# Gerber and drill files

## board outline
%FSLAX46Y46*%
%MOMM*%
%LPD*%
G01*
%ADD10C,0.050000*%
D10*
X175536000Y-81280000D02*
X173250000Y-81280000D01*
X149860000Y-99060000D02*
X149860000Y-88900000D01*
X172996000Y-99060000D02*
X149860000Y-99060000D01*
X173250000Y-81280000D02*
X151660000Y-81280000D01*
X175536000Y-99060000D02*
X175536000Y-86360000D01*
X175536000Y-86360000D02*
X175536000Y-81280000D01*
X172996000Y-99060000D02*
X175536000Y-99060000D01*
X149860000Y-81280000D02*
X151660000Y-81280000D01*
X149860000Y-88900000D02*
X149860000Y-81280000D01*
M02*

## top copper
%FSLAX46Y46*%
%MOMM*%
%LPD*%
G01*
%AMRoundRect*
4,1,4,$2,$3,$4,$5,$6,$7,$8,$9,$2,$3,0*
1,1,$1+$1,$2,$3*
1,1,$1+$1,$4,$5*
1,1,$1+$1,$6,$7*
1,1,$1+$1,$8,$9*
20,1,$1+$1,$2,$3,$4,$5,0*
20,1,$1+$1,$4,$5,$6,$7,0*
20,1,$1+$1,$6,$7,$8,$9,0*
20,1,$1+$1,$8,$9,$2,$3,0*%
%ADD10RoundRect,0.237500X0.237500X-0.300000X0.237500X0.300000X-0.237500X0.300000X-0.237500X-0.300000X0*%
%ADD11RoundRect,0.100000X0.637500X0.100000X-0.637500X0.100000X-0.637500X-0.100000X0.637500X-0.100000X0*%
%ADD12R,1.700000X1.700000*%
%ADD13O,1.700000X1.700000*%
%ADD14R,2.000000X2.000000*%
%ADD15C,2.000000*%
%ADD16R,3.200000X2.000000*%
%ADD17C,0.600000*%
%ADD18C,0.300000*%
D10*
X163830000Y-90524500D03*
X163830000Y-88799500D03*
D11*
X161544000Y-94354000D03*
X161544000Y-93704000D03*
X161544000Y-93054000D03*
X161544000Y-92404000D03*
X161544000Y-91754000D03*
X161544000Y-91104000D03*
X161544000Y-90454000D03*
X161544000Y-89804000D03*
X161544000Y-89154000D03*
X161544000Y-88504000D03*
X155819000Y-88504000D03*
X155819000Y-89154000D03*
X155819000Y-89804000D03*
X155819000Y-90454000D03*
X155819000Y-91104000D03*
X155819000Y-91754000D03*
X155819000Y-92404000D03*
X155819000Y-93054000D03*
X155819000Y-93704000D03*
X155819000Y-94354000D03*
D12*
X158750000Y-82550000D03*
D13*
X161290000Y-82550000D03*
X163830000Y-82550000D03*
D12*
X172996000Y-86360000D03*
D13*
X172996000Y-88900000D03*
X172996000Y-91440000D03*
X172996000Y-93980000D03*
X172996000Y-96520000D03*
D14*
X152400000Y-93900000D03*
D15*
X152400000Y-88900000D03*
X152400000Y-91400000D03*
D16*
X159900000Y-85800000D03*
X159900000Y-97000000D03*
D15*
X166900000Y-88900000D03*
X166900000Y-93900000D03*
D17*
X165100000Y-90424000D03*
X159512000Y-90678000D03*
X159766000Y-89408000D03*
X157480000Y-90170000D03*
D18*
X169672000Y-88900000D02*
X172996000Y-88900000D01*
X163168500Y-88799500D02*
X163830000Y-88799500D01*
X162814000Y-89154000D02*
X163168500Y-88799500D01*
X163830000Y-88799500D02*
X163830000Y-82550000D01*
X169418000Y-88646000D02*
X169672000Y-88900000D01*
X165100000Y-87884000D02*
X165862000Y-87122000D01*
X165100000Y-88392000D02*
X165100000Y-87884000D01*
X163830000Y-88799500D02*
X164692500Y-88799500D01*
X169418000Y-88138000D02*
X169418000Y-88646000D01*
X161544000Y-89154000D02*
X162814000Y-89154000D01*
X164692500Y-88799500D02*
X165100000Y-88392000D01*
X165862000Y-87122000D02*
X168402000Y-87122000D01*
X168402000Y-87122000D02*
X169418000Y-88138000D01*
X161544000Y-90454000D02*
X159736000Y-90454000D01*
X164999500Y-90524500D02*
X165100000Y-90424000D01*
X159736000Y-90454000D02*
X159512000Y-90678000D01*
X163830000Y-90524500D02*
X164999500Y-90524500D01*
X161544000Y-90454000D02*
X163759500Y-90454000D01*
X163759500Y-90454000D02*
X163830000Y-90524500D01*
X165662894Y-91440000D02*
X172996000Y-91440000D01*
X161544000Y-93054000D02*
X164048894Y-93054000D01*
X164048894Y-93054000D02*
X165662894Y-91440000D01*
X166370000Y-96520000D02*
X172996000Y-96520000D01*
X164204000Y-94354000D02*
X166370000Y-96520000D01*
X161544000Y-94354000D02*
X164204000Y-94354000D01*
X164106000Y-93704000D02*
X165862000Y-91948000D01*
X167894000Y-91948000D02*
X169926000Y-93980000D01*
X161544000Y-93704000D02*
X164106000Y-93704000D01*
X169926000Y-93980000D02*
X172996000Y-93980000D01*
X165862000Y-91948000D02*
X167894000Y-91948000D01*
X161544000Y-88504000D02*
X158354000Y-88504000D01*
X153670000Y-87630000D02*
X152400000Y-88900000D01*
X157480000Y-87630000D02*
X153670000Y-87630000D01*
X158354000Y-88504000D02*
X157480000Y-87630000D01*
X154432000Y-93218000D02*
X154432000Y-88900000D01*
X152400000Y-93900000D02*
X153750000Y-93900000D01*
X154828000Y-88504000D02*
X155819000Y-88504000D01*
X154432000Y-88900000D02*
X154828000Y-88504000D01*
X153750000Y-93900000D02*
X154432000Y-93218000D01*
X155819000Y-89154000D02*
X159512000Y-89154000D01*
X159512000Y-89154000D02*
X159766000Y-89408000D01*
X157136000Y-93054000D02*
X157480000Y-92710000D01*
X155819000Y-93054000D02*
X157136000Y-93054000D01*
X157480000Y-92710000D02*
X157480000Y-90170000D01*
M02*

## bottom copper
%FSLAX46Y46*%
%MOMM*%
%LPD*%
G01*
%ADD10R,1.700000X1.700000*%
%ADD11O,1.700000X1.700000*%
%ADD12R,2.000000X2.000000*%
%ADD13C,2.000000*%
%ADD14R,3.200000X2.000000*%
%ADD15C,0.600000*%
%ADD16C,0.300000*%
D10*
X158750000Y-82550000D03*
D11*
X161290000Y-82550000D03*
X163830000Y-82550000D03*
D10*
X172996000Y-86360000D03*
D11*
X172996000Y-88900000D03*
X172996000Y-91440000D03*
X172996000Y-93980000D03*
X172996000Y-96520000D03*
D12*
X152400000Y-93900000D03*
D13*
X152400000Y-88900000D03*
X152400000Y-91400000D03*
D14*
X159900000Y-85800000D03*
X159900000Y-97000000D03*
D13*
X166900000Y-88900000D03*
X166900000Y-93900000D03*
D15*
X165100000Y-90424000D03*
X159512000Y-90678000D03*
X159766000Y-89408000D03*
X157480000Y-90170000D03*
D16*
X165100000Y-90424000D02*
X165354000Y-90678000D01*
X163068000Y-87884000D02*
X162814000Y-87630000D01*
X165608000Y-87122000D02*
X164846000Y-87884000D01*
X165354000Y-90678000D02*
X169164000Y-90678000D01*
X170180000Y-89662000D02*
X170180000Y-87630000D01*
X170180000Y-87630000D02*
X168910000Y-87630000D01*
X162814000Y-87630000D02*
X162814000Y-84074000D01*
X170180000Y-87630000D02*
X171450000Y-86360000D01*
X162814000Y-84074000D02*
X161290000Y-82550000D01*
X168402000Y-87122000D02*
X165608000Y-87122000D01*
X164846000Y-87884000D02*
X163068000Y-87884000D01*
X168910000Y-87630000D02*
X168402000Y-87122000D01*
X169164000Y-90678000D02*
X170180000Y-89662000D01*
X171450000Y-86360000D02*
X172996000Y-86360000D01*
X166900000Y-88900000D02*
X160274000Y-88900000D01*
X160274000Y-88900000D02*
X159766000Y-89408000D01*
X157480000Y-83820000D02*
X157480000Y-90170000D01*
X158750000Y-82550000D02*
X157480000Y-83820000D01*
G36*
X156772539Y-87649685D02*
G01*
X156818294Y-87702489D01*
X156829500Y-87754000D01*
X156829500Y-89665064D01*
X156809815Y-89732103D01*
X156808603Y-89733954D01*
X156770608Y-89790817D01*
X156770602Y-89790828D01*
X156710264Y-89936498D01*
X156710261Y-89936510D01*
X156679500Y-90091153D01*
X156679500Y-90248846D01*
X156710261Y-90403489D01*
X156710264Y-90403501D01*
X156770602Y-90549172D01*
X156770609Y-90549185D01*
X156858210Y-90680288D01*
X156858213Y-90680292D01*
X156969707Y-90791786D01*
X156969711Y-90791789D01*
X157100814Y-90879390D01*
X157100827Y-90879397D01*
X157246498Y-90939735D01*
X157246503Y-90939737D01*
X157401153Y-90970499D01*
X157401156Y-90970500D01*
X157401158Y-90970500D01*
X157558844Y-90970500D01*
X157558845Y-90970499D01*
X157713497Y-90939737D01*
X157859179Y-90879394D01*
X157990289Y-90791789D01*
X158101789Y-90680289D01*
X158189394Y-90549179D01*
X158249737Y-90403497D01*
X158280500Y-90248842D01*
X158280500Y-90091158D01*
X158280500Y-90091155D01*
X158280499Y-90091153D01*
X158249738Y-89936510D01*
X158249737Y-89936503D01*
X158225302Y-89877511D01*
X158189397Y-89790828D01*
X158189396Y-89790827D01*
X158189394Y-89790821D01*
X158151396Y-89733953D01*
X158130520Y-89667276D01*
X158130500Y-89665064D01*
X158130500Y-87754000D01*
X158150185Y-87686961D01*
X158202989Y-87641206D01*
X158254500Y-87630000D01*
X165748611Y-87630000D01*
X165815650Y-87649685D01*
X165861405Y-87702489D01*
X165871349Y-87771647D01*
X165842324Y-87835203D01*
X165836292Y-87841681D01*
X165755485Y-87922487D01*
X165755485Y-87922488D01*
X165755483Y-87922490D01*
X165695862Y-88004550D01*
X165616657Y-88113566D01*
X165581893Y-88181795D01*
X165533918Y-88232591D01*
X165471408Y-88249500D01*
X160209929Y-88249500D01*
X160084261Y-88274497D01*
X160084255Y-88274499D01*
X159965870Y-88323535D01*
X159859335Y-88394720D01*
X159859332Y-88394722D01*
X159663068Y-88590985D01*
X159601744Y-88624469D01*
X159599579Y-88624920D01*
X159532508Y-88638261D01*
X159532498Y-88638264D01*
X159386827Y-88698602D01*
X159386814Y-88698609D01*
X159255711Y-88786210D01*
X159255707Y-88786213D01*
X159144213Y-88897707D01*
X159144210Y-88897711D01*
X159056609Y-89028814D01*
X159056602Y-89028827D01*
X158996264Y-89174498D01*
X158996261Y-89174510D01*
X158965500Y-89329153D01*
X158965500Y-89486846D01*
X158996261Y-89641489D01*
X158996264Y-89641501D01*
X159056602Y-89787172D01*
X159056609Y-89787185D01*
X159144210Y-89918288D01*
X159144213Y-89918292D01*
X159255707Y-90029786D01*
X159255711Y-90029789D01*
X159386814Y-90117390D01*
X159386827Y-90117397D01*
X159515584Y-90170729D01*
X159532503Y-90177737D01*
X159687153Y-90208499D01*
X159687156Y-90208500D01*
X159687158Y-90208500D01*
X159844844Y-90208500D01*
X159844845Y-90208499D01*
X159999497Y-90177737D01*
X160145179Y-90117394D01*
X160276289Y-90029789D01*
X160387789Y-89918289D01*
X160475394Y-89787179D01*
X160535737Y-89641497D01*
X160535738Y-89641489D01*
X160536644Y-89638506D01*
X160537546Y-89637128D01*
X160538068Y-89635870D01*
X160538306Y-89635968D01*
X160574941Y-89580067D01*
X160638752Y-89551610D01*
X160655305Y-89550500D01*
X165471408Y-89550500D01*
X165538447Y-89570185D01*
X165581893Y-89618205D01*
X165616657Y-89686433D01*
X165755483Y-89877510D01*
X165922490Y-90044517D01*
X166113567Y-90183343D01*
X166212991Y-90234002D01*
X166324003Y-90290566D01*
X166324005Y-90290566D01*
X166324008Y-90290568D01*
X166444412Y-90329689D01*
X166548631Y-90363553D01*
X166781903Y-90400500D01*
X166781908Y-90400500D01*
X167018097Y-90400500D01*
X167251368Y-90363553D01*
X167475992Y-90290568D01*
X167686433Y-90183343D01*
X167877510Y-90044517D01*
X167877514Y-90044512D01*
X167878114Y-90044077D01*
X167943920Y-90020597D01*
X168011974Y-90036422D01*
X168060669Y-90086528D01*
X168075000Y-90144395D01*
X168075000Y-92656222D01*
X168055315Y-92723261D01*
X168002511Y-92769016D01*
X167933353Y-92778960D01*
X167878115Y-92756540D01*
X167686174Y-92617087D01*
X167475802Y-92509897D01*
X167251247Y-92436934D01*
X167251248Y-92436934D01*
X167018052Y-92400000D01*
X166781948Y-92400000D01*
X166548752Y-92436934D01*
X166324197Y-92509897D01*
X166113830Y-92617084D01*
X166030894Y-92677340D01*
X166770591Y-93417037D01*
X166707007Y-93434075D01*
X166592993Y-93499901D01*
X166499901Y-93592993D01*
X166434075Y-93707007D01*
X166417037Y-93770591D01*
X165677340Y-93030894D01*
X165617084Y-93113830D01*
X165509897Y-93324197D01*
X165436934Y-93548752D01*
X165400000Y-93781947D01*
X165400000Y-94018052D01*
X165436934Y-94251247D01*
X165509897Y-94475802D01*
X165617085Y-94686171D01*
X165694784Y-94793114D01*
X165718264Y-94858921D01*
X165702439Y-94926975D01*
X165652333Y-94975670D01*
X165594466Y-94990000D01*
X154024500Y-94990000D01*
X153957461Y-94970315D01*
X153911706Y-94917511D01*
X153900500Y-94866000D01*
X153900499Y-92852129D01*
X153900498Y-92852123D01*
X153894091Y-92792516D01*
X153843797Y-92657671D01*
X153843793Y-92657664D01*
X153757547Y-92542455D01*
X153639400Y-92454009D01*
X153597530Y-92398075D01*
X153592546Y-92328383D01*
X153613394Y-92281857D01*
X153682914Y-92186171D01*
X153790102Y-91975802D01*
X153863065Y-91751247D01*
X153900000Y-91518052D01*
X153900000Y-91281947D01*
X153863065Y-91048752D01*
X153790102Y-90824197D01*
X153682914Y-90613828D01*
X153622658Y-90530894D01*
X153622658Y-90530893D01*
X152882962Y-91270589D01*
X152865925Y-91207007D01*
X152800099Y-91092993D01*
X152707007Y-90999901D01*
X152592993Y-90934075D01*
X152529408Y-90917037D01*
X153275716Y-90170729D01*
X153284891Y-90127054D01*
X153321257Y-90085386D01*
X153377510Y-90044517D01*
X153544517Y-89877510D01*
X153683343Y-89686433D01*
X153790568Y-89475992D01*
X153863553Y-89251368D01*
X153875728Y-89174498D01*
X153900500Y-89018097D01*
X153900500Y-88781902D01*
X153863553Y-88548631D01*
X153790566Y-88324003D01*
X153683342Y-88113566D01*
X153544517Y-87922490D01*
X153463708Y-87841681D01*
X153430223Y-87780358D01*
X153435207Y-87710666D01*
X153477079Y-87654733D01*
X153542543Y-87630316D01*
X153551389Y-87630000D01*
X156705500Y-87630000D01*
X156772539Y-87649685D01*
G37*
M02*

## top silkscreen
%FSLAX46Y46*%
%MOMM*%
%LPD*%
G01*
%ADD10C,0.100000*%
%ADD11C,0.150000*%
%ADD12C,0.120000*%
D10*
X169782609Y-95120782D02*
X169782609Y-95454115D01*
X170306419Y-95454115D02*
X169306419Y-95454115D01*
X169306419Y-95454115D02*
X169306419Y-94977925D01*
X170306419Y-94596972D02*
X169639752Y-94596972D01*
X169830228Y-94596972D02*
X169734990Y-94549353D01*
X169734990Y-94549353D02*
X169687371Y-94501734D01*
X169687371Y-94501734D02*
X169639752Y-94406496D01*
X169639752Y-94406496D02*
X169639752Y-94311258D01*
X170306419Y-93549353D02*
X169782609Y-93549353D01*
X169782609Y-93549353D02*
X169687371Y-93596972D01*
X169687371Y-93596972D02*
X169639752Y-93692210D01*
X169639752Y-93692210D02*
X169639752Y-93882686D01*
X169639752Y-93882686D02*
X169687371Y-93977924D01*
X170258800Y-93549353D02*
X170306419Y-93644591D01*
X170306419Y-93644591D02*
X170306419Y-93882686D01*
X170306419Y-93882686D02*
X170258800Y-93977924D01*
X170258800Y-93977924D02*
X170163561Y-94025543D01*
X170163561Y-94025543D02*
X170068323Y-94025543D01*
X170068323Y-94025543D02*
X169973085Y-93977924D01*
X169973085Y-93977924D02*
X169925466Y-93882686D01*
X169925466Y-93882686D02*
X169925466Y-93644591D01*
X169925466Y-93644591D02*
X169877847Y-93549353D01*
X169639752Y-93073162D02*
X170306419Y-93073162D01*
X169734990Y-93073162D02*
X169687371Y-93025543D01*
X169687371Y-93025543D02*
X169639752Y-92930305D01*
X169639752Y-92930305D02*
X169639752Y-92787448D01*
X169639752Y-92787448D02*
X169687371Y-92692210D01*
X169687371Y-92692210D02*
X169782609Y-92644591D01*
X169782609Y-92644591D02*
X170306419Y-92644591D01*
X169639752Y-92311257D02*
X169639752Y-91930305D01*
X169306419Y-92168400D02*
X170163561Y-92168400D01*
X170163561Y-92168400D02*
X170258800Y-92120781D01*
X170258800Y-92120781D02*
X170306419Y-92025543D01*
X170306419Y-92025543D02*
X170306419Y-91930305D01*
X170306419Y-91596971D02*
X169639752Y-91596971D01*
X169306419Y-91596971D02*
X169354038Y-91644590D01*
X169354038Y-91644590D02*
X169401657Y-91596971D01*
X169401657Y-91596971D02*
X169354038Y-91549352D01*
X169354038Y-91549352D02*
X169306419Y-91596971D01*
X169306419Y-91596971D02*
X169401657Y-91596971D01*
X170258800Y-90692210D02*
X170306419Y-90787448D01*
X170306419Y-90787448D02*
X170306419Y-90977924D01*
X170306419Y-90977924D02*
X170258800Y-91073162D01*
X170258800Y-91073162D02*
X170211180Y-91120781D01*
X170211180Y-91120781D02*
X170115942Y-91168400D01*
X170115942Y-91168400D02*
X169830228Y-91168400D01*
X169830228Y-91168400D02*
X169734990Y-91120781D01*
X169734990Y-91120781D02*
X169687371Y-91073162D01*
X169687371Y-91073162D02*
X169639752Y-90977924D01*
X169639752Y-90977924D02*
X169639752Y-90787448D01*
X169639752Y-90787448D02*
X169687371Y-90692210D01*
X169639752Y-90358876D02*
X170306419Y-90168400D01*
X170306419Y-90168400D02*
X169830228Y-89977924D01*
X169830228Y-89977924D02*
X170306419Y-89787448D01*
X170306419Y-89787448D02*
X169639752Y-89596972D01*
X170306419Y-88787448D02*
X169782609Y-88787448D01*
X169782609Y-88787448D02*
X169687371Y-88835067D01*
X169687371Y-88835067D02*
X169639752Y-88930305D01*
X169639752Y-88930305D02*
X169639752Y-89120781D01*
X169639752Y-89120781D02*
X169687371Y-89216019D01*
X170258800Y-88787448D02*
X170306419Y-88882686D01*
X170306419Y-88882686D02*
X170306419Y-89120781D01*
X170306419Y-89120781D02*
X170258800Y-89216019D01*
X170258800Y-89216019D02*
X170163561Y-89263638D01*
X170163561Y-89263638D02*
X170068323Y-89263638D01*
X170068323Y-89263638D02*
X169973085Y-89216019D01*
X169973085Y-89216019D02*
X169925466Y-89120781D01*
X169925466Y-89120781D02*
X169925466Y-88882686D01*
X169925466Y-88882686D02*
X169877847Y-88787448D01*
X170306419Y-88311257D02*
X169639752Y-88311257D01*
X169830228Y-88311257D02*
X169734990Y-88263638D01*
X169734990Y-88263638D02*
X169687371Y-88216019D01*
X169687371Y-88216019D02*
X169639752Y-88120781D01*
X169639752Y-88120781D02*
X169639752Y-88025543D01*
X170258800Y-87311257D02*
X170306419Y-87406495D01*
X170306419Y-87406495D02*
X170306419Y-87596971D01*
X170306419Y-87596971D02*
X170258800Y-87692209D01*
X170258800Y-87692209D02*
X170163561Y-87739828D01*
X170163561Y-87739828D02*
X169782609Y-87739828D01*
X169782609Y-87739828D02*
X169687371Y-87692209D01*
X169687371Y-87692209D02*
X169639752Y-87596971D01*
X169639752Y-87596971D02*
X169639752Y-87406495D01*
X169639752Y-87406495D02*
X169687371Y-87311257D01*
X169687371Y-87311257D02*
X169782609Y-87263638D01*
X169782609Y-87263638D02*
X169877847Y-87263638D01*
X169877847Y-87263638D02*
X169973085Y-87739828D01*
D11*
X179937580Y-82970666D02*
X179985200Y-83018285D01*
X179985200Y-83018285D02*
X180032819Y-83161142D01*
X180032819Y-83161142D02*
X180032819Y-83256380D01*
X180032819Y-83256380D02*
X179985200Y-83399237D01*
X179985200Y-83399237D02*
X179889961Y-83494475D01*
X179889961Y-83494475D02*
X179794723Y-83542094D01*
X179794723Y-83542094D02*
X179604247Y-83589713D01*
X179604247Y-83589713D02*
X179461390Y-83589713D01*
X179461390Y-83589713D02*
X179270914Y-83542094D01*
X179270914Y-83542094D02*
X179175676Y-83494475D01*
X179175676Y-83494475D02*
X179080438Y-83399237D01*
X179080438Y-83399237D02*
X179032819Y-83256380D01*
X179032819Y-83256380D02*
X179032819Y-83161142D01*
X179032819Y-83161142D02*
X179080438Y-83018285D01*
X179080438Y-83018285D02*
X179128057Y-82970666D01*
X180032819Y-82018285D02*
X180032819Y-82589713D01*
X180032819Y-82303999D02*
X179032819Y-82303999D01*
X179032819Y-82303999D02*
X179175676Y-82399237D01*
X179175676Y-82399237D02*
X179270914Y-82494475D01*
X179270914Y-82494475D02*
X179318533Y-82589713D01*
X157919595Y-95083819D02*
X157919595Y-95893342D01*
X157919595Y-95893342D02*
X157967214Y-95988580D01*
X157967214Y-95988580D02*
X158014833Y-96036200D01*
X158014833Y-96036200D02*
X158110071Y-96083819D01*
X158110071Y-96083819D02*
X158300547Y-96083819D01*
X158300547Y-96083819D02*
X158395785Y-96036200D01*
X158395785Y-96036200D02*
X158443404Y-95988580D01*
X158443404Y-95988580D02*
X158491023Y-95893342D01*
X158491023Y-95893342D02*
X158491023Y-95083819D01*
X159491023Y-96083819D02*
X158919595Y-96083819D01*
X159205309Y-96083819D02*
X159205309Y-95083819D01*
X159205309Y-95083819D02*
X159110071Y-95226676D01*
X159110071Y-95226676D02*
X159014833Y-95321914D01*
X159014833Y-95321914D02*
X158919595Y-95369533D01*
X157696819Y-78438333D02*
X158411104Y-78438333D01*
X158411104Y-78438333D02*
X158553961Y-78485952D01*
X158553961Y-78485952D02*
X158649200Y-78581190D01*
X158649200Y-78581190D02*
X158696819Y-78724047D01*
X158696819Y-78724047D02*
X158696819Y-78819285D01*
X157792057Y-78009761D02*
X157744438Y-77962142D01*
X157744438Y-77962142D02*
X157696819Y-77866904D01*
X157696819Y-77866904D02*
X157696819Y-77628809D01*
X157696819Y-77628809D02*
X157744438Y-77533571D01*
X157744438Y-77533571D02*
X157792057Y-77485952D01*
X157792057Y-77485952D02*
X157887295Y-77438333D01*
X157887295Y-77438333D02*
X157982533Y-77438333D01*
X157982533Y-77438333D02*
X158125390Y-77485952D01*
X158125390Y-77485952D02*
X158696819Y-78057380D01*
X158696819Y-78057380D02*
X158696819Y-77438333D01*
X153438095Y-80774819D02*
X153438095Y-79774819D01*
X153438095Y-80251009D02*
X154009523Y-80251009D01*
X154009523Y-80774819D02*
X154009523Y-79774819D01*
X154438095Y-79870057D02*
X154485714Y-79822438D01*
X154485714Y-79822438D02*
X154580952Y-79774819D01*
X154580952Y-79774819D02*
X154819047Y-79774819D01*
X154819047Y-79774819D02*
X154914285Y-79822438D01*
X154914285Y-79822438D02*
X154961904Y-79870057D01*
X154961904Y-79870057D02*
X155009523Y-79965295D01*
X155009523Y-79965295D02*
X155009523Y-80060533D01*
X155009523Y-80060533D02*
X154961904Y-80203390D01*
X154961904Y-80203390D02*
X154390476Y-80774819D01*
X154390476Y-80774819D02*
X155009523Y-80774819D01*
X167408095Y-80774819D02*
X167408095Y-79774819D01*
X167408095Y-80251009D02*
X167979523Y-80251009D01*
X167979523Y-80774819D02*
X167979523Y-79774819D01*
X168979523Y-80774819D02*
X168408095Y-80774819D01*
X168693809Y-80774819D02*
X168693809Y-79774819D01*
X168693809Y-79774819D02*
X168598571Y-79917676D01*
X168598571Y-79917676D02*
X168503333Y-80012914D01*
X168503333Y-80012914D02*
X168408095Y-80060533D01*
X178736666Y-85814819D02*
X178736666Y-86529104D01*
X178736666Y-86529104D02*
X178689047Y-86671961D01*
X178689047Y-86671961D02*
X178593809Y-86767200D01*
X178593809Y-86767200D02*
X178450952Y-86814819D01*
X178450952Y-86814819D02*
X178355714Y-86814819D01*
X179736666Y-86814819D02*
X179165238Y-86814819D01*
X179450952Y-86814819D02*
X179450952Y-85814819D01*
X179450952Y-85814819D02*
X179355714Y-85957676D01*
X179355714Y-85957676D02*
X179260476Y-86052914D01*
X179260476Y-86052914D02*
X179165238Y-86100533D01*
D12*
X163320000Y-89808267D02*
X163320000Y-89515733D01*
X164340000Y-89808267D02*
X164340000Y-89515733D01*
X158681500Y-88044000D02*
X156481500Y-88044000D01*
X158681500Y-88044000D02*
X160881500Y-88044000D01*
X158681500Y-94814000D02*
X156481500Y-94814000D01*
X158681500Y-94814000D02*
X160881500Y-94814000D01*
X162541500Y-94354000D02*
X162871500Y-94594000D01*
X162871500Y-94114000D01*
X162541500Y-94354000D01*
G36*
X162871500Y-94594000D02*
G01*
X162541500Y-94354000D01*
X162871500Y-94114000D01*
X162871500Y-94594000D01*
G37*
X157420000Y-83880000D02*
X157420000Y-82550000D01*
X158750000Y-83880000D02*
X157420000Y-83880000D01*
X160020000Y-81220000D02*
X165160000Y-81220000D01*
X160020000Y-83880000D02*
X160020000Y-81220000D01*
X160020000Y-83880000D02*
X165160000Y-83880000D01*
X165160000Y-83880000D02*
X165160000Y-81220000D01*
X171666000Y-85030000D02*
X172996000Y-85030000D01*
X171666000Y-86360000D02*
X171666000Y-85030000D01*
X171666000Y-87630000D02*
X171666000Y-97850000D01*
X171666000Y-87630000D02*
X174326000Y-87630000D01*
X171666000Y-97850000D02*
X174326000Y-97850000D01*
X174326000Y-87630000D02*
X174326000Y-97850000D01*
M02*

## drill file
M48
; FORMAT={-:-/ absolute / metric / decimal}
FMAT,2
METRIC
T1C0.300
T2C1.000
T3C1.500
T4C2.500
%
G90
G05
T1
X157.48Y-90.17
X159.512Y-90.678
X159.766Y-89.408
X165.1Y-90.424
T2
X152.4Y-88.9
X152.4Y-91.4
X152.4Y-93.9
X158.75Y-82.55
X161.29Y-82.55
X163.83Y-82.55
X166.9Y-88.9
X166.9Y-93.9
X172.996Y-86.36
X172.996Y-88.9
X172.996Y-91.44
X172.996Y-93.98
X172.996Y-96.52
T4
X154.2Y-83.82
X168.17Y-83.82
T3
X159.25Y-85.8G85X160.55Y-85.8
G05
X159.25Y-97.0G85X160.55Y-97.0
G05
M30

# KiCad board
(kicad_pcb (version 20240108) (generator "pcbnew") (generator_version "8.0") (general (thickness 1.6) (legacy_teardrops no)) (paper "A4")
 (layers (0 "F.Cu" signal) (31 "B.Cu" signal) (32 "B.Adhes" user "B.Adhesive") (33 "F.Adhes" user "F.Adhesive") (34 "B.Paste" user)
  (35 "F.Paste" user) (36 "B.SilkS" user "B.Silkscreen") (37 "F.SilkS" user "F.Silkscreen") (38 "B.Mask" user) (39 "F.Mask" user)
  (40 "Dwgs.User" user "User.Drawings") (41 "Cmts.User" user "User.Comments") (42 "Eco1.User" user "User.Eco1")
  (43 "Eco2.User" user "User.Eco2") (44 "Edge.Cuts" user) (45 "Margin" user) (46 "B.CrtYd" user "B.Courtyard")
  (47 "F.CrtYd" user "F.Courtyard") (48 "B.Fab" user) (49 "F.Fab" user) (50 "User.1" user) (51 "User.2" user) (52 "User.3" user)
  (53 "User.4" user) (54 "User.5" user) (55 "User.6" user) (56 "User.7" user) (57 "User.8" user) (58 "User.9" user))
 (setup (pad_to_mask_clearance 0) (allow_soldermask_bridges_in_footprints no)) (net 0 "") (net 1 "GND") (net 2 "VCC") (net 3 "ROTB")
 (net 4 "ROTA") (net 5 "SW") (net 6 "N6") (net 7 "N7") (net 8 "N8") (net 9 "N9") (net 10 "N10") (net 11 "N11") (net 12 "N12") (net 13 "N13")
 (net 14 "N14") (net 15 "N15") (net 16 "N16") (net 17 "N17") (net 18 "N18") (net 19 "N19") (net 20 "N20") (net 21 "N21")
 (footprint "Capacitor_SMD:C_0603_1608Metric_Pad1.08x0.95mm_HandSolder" (layer "F.Cu") (at 163.83 89.662 90)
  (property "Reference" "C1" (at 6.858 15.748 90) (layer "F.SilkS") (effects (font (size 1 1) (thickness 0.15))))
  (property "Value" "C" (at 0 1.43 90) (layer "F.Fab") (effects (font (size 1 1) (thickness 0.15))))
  (fp_line (start -0.146267 -0.51) (end 0.146267 -0.51) (stroke (width 0.12) (type solid)) (layer "F.SilkS"))
  (fp_line (start -0.146267 0.51) (end 0.146267 0.51) (stroke (width 0.12) (type solid)) (layer "F.SilkS"))
  (pad "1" smd roundrect (at -0.8625 0 90) (size 1.075 0.95) (layers "F.Cu" "F.Paste" "F.Mask") (roundrect_rratio 0.25) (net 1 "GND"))
  (pad "2" smd roundrect (at 0.8625 0 90) (size 1.075 0.95) (layers "F.Cu" "F.Paste" "F.Mask") (roundrect_rratio 0.25) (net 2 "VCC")))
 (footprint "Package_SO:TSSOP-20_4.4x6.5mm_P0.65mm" (layer "F.Cu") (at 158.6815 91.429 180)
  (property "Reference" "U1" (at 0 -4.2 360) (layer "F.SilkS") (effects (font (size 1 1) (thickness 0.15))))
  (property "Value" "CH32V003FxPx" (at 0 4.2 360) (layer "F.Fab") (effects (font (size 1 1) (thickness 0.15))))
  (fp_line (start 0 3.385) (end 2.2 3.385) (stroke (width 0.12) (type solid)) (layer "F.SilkS"))
  (fp_line (start 0 3.385) (end -2.2 3.385) (stroke (width 0.12) (type solid)) (layer "F.SilkS"))
  (fp_line (start 0 -3.385) (end 2.2 -3.385) (stroke (width 0.12) (type solid)) (layer "F.SilkS"))
  (fp_line (start 0 -3.385) (end -2.2 -3.385) (stroke (width 0.12) (type solid)) (layer "F.SilkS"))
  (fp_poly
   (pts (xy -3.86 -2.925) (xy -4.19 -3.165) (xy -4.19 -2.685) (xy -3.86 -2.925)) (stroke (width 0.12) (type solid)) (fill solid)
   (layer "F.SilkS"))
  (pad "1" smd roundrect (at -2.8625 -2.925 180) (size 1.475 0.4) (layers "F.Cu" "F.Paste" "F.Mask") (roundrect_rratio 0.25) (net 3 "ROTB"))
  (pad "2" smd roundrect (at -2.8625 -2.275 180) (size 1.475 0.4) (layers "F.Cu" "F.Paste" "F.Mask") (roundrect_rratio 0.25) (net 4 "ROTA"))
  (pad "3" smd roundrect (at -2.8625 -1.625 180) (size 1.475 0.4) (layers "F.Cu" "F.Paste" "F.Mask") (roundrect_rratio 0.25) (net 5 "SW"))
  (pad "4" smd roundrect (at -2.8625 -0.975 180) (size 1.475 0.4) (layers "F.Cu" "F.Paste" "F.Mask") (roundrect_rratio 0.25) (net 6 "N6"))
  (pad "5" smd roundrect (at -2.8625 -0.325 180) (size 1.475 0.4) (layers "F.Cu" "F.Paste" "F.Mask") (roundrect_rratio 0.25) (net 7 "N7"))
  (pad "6" smd roundrect (at -2.8625 0.325 180) (size 1.475 0.4) (layers "F.Cu" "F.Paste" "F.Mask") (roundrect_rratio 0.25) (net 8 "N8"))
  (pad "7" smd roundrect (at -2.8625 0.975 180) (size 1.475 0.4) (layers "F.Cu" "F.Paste" "F.Mask") (roundrect_rratio 0.25) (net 1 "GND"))
  (pad "8" smd roundrect (at -2.8625 1.625 180) (size 1.475 0.4) (layers "F.Cu" "F.Paste" "F.Mask") (roundrect_rratio 0.25) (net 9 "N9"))
  (pad "9" smd roundrect (at -2.8625 2.275 180) (size 1.475 0.4) (layers "F.Cu" "F.Paste" "F.Mask") (roundrect_rratio 0.25) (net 2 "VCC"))
  (pad "10" smd roundrect (at -2.8625 2.925 180) (size 1.475 0.4) (layers "F.Cu" "F.Paste" "F.Mask") (roundrect_rratio 0.25) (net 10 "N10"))
  (pad "11" smd roundrect (at 2.8625 2.925 180) (size 1.475 0.4) (layers "F.Cu" "F.Paste" "F.Mask") (roundrect_rratio 0.25) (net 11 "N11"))
  (pad "12" smd roundrect (at 2.8625 2.275 180) (size 1.475 0.4) (layers "F.Cu" "F.Paste" "F.Mask") (roundrect_rratio 0.25) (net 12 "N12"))
  (pad "13" smd roundrect (at 2.8625 1.625 180) (size 1.475 0.4) (layers "F.Cu" "F.Paste" "F.Mask") (roundrect_rratio 0.25) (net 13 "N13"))
  (pad "14" smd roundrect (at 2.8625 0.975 180) (size 1.475 0.4) (layers "F.Cu" "F.Paste" "F.Mask") (roundrect_rratio 0.25) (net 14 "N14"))
  (pad "15" smd roundrect (at 2.8625 0.325 180) (size 1.475 0.4) (layers "F.Cu" "F.Paste" "F.Mask") (roundrect_rratio 0.25) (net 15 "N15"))
  (pad "16" smd roundrect (at 2.8625 -0.325 180) (size 1.475 0.4) (layers "F.Cu" "F.Paste" "F.Mask") (roundrect_rratio 0.25) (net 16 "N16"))
  (pad "17" smd roundrect (at 2.8625 -0.975 180) (size 1.475 0.4) (layers "F.Cu" "F.Paste" "F.Mask") (roundrect_rratio 0.25) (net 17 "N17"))
  (pad "18" smd roundrect (at 2.8625 -1.625 180) (size 1.475 0.4) (layers "F.Cu" "F.Paste" "F.Mask") (roundrect_rratio 0.25) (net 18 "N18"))
  (pad "19" smd roundrect (at 2.8625 -2.275 180) (size 1.475 0.4) (layers "F.Cu" "F.Paste" "F.Mask") (roundrect_rratio 0.25) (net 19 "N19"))
  (pad "20" smd roundrect (at 2.8625 -2.925 180) (size 1.475 0.4) (layers "F.Cu" "F.Paste" "F.Mask") (roundrect_rratio 0.25) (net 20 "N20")))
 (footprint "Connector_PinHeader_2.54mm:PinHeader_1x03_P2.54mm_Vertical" (layer "F.Cu") (at 158.75 82.55 90)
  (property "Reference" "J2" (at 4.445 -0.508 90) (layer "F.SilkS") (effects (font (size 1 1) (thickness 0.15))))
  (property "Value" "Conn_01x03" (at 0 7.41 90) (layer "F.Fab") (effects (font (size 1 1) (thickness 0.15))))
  (fp_line (start -1.33 -1.33) (end 0 -1.33) (stroke (width 0.12) (type solid)) (layer "F.SilkS"))
  (fp_line (start -1.33 0) (end -1.33 -1.33) (stroke (width 0.12) (type solid)) (layer "F.SilkS"))
  (fp_line (start 1.33 1.27) (end 1.33 6.41) (stroke (width 0.12) (type solid)) (layer "F.SilkS"))
  (fp_line (start -1.33 1.27) (end 1.33 1.27) (stroke (width 0.12) (type solid)) (layer "F.SilkS"))
  (fp_line (start -1.33 1.27) (end -1.33 6.41) (stroke (width 0.12) (type solid)) (layer "F.SilkS"))
  (fp_line (start -1.33 6.41) (end 1.33 6.41) (stroke (width 0.12) (type solid)) (layer "F.SilkS"))
  (pad "1" thru_hole rect (at 0 0 90) (size 1.7 1.7) (drill 1) (layers "*.Cu" "*.Mask") (remove_unused_layers no) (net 18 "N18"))
  (pad "2" thru_hole oval (at 0 2.54 90) (size 1.7 1.7) (drill 1) (layers "*.Cu" "*.Mask") (remove_unused_layers no) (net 1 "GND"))
  (pad "3" thru_hole oval (at 0 5.08 90) (size 1.7 1.7) (drill 1) (layers "*.Cu" "*.Mask") (remove_unused_layers no) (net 2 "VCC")))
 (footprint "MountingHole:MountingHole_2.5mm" (layer "F.Cu") (at 154.2 83.82)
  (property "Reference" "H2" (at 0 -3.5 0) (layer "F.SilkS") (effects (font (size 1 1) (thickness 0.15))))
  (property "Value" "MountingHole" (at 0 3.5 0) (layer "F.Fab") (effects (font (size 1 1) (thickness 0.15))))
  (pad "" np_thru_hole circle (at 0 0) (size 2.5 2.5) (drill 2.5) (layers "*.Cu" "*.Mask")))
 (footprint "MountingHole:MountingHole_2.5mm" (layer "F.Cu") (at 168.17 83.82)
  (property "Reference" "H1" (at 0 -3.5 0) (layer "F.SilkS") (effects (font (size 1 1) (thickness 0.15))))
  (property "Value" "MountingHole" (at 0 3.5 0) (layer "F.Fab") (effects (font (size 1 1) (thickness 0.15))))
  (pad "" np_thru_hole circle (at 0 0) (size 2.5 2.5) (drill 2.5) (layers "*.Cu" "*.Mask")))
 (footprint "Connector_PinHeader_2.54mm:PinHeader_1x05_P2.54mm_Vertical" (layer "F.Cu") (at 172.996 86.36)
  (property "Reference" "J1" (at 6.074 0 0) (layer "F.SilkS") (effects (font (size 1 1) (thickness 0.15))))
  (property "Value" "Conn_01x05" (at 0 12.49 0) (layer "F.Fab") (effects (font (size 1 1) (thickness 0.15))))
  (fp_line (start -1.33 -1.33) (end 0 -1.33) (stroke (width 0.12) (type solid)) (layer "F.SilkS"))
  (fp_line (start -1.33 0) (end -1.33 -1.33) (stroke (width 0.12) (type solid)) (layer "F.SilkS"))
  (fp_line (start -1.33 1.27) (end -1.33 11.49) (stroke (width 0.12) (type solid)) (layer "F.SilkS"))
  (fp_line (start -1.33 1.27) (end 1.33 1.27) (stroke (width 0.12) (type solid)) (layer "F.SilkS"))
  (fp_line (start -1.33 11.49) (end 1.33 11.49) (stroke (width 0.12) (type solid)) (layer "F.SilkS"))
  (fp_line (start 1.33 1.27) (end 1.33 11.49) (stroke (width 0.12) (type solid)) (layer "F.SilkS"))
  (pad "1" thru_hole rect (at 0 0) (size 1.7 1.7) (drill 1) (layers "*.Cu" "*.Mask") (remove_unused_layers no) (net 1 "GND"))
  (pad "2" thru_hole oval (at 0 2.54) (size 1.7 1.7) (drill 1) (layers "*.Cu" "*.Mask") (remove_unused_layers no) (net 2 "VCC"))
  (pad "3" thru_hole oval (at 0 5.08) (size 1.7 1.7) (drill 1) (layers "*.Cu" "*.Mask") (remove_unused_layers no) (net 5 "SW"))
  (pad "4" thru_hole oval (at 0 7.62) (size 1.7 1.7) (drill 1) (layers "*.Cu" "*.Mask") (remove_unused_layers no) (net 4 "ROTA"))
  (pad "5" thru_hole oval (at 0 10.16) (size 1.7 1.7) (drill 1) (layers "*.Cu" "*.Mask") (remove_unused_layers no) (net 3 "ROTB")))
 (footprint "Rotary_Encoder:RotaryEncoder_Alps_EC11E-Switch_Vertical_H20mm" (layer "B.Cu") (at 152.4 93.9)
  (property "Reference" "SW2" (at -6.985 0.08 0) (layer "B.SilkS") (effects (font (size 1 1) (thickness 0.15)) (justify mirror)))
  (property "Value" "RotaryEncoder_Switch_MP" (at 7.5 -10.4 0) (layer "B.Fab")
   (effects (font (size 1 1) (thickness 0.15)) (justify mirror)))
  (pad "A" thru_hole rect (at 0 0) (size 2 2) (drill 1) (layers "*.Cu" "*.Mask") (remove_unused_layers no) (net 11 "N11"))
  (pad "B" thru_hole circle (at 0 -5) (size 2 2) (drill 1) (layers "*.Cu" "*.Mask") (remove_unused_layers no) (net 10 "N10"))
  (pad "C" thru_hole circle (at 0 -2.5) (size 2 2) (drill 1) (layers "*.Cu" "*.Mask") (remove_unused_layers no) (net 1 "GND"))
  (pad "MP" thru_hole rect (at 7.5 -8.1) (size 3.2 2) (drill oval 2.8 1.5) (layers "*.Cu" "*.Mask") (remove_unused_layers no) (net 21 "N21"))
  (pad "MP" thru_hole rect (at 7.5 3.1) (size 3.2 2) (drill oval 2.8 1.5) (layers "*.Cu" "*.Mask") (remove_unused_layers no) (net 21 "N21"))
  (pad "S1" thru_hole circle (at 14.5 -5) (size 2 2) (drill 1) (layers "*.Cu" "*.Mask") (remove_unused_layers no) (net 12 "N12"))
  (pad "S2" thru_hole circle (at 14.5 0) (size 2 2) (drill 1) (layers "*.Cu" "*.Mask") (remove_unused_layers no) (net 1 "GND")))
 (gr_line (start 175.536 81.28) (end 173.25 81.28) (stroke (width 0.05) (type default)) (layer "Edge.Cuts"))
 (gr_line (start 149.86 99.06) (end 149.86 88.9) (stroke (width 0.05) (type default)) (layer "Edge.Cuts"))
 (gr_line (start 172.996 99.06) (end 149.86 99.06) (stroke (width 0.05) (type default)) (layer "Edge.Cuts"))
 (gr_line (start 173.25 81.28) (end 151.66 81.28) (stroke (width 0.05) (type default)) (layer "Edge.Cuts"))
 (gr_line (start 175.536 99.06) (end 175.536 86.36) (stroke (width 0.05) (type default)) (layer "Edge.Cuts"))
 (gr_line (start 175.536 86.36) (end 175.536 81.28) (stroke (width 0.05) (type default)) (layer "Edge.Cuts"))
 (gr_line (start 172.996 99.06) (end 175.536 99.06) (stroke (width 0.05) (type default)) (layer "Edge.Cuts"))
 (gr_line (start 149.86 81.28) (end 151.66 81.28) (stroke (width 0.05) (type default)) (layer "Edge.Cuts"))
 (gr_line (start 149.86 88.9) (end 149.86 81.28) (stroke (width 0.05) (type default)) (layer "Edge.Cuts"))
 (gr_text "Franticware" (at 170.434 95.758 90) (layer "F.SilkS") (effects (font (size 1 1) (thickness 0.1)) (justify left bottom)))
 (segment (start 169.672 88.9) (end 172.996 88.9) (width 0.3) (layer "F.Cu") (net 2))
 (segment (start 163.1685 88.7995) (end 163.83 88.7995) (width 0.3) (layer "F.Cu") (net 2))
 (segment (start 162.814 89.154) (end 163.1685 88.7995) (width 0.3) (layer "F.Cu") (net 2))
 (segment (start 163.83 88.7995) (end 163.83 82.55) (width 0.3) (layer "F.Cu") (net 2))
 (segment (start 169.418 88.646) (end 169.672 88.9) (width 0.3) (layer "F.Cu") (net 2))
 (segment (start 165.1 87.884) (end 165.862 87.122) (width 0.3) (layer "F.Cu") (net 2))
 (segment (start 165.1 88.392) (end 165.1 87.884) (width 0.3) (layer "F.Cu") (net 2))
 (segment (start 163.83 88.7995) (end 164.6925 88.7995) (width 0.3) (layer "F.Cu") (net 2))
 (segment (start 169.418 88.138) (end 169.418 88.646) (width 0.3) (layer "F.Cu") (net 2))
 (segment (start 161.544 89.154) (end 162.814 89.154) (width 0.3) (layer "F.Cu") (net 2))
 (segment (start 164.6925 88.7995) (end 165.1 88.392) (width 0.3) (layer "F.Cu") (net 2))
 (segment (start 165.862 87.122) (end 168.402 87.122) (width 0.3) (layer "F.Cu") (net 2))
 (segment (start 168.402 87.122) (end 169.418 88.138) (width 0.3) (layer "F.Cu") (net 2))
 (segment (start 161.544 90.454) (end 159.736 90.454) (width 0.3) (layer "F.Cu") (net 1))
 (segment (start 164.9995 90.5245) (end 165.1 90.424) (width 0.3) (layer "F.Cu") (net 1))
 (segment (start 159.736 90.454) (end 159.512 90.678) (width 0.3) (layer "F.Cu") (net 1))
 (segment (start 163.83 90.5245) (end 164.9995 90.5245) (width 0.3) (layer "F.Cu") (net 1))
 (segment (start 161.544 90.454) (end 163.7595 90.454) (width 0.3) (layer "F.Cu") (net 1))
 (segment (start 163.7595 90.454) (end 163.83 90.5245) (width 0.3) (layer "F.Cu") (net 1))
 (via (at 165.1 90.424) (size 0.6) (drill 0.3) (layers "F.Cu" "B.Cu") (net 1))
 (via (at 159.512 90.678) (size 0.6) (drill 0.3) (layers "F.Cu" "B.Cu") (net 1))
 (segment (start 165.1 90.424) (end 165.354 90.678) (width 0.3) (layer "B.Cu") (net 1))
 (segment (start 163.068 87.884) (end 162.814 87.63) (width 0.3) (layer "B.Cu") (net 1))
 (segment (start 165.608 87.122) (end 164.846 87.884) (width 0.3) (layer "B.Cu") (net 1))
 (segment (start 165.354 90.678) (end 169.164 90.678) (width 0.3) (layer "B.Cu") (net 1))
 (segment (start 170.18 89.662) (end 170.18 87.63) (width 0.3) (layer "B.Cu") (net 1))
 (segment (start 170.18 87.63) (end 168.91 87.63) (width 0.3) (layer "B.Cu") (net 1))
 (segment (start 162.814 87.63) (end 162.814 84.074) (width 0.3) (layer "B.Cu") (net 1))
 (segment (start 170.18 87.63) (end 171.45 86.36) (width 0.3) (layer "B.Cu") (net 1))
 (segment (start 162.814 84.074) (end 161.29 82.55) (width 0.3) (layer "B.Cu") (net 1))
 (segment (start 168.402 87.122) (end 165.608 87.122) (width 0.3) (layer "B.Cu") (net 1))
 (segment (start 164.846 87.884) (end 163.068 87.884) (width 0.3) (layer "B.Cu") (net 1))
 (segment (start 168.91 87.63) (end 168.402 87.122) (width 0.3) (layer "B.Cu") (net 1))
 (segment (start 169.164 90.678) (end 170.18 89.662) (width 0.3) (layer "B.Cu") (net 1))
 (segment (start 171.45 86.36) (end 172.996 86.36) (width 0.3) (layer "B.Cu") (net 1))
 (segment (start 165.662894 91.44) (end 172.996 91.44) (width 0.3) (layer "F.Cu") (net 5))
 (segment (start 161.544 93.054) (end 164.048894 93.054) (width 0.3) (layer "F.Cu") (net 5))
 (segment (start 164.048894 93.054) (end 165.662894 91.44) (width 0.3) (layer "F.Cu") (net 5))
 (segment (start 166.37 96.52) (end 172.996 96.52) (width 0.3) (layer "F.Cu") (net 3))
 (segment (start 164.204 94.354) (end 166.37 96.52) (width 0.3) (layer "F.Cu") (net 3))
 (segment (start 161.544 94.354) (end 164.204 94.354) (width 0.3) (layer "F.Cu") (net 3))
 (segment (start 164.106 93.704) (end 165.862 91.948) (width 0.3) (layer "F.Cu") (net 4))
 (segment (start 167.894 91.948) (end 169.926 93.98) (width 0.3) (layer "F.Cu") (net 4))
 (segment (start 161.544 93.704) (end 164.106 93.704) (width 0.3) (layer "F.Cu") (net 4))
 (segment (start 169.926 93.98) (end 172.996 93.98) (width 0.3) (layer "F.Cu") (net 4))
 (segment (start 165.862 91.948) (end 167.894 91.948) (width 0.3) (layer "F.Cu") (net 4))
 (segment (start 161.544 88.504) (end 158.354 88.504) (width 0.3) (layer "F.Cu") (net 10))
 (segment (start 153.67 87.63) (end 152.4 88.9) (width 0.3) (layer "F.Cu") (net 10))
 (segment (start 157.48 87.63) (end 153.67 87.63) (width 0.3) (layer "F.Cu") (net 10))
 (segment (start 158.354 88.504) (end 157.48 87.63) (width 0.3) (layer "F.Cu") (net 10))
 (segment (start 154.432 93.218) (end 154.432 88.9) (width 0.3) (layer "F.Cu") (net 11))
 (segment (start 152.4 93.9) (end 153.75 93.9) (width 0.3) (layer "F.Cu") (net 11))
 (segment (start 154.828 88.504) (end 155.819 88.504) (width 0.3) (layer "F.Cu") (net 11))
 (segment (start 154.432 88.9) (end 154.828 88.504) (width 0.3) (layer "F.Cu") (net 11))
 (segment (start 153.75 93.9) (end 154.432 93.218) (width 0.3) (layer "F.Cu") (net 11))
 (segment (start 155.819 89.154) (end 159.512 89.154) (width 0.3) (layer "F.Cu") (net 12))
 (segment (start 159.512 89.154) (end 159.766 89.408) (width 0.3) (layer "F.Cu") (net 12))
 (via (at 159.766 89.408) (size 0.6) (drill 0.3) (layers "F.Cu" "B.Cu") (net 12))
 (segment (start 166.9 88.9) (end 160.274 88.9) (width 0.3) (layer "B.Cu") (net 12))
 (segment (start 160.274 88.9) (end 159.766 89.408) (width 0.3) (layer "B.Cu") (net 12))
 (segment (start 157.136 93.054) (end 157.48 92.71) (width 0.3) (layer "F.Cu") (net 18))
 (segment (start 155.819 93.054) (end 157.136 93.054) (width 0.3) (layer "F.Cu") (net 18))
 (segment (start 157.48 92.71) (end 157.48 90.17) (width 0.3) (layer "F.Cu") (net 18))
 (via (at 157.48 90.17) (size 0.6) (drill 0.3) (layers "F.Cu" "B.Cu") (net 18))
 (segment (start 157.48 83.82) (end 157.48 90.17) (width 0.3) (layer "B.Cu") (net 18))
 (segment (start 158.75 82.55) (end 157.48 83.82) (width 0.3) (layer "B.Cu") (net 18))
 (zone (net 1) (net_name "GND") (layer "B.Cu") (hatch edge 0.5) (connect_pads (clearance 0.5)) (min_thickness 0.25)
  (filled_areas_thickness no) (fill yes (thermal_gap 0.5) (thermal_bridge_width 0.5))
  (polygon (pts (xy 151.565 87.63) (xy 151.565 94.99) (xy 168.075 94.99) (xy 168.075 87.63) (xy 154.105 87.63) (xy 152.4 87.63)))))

